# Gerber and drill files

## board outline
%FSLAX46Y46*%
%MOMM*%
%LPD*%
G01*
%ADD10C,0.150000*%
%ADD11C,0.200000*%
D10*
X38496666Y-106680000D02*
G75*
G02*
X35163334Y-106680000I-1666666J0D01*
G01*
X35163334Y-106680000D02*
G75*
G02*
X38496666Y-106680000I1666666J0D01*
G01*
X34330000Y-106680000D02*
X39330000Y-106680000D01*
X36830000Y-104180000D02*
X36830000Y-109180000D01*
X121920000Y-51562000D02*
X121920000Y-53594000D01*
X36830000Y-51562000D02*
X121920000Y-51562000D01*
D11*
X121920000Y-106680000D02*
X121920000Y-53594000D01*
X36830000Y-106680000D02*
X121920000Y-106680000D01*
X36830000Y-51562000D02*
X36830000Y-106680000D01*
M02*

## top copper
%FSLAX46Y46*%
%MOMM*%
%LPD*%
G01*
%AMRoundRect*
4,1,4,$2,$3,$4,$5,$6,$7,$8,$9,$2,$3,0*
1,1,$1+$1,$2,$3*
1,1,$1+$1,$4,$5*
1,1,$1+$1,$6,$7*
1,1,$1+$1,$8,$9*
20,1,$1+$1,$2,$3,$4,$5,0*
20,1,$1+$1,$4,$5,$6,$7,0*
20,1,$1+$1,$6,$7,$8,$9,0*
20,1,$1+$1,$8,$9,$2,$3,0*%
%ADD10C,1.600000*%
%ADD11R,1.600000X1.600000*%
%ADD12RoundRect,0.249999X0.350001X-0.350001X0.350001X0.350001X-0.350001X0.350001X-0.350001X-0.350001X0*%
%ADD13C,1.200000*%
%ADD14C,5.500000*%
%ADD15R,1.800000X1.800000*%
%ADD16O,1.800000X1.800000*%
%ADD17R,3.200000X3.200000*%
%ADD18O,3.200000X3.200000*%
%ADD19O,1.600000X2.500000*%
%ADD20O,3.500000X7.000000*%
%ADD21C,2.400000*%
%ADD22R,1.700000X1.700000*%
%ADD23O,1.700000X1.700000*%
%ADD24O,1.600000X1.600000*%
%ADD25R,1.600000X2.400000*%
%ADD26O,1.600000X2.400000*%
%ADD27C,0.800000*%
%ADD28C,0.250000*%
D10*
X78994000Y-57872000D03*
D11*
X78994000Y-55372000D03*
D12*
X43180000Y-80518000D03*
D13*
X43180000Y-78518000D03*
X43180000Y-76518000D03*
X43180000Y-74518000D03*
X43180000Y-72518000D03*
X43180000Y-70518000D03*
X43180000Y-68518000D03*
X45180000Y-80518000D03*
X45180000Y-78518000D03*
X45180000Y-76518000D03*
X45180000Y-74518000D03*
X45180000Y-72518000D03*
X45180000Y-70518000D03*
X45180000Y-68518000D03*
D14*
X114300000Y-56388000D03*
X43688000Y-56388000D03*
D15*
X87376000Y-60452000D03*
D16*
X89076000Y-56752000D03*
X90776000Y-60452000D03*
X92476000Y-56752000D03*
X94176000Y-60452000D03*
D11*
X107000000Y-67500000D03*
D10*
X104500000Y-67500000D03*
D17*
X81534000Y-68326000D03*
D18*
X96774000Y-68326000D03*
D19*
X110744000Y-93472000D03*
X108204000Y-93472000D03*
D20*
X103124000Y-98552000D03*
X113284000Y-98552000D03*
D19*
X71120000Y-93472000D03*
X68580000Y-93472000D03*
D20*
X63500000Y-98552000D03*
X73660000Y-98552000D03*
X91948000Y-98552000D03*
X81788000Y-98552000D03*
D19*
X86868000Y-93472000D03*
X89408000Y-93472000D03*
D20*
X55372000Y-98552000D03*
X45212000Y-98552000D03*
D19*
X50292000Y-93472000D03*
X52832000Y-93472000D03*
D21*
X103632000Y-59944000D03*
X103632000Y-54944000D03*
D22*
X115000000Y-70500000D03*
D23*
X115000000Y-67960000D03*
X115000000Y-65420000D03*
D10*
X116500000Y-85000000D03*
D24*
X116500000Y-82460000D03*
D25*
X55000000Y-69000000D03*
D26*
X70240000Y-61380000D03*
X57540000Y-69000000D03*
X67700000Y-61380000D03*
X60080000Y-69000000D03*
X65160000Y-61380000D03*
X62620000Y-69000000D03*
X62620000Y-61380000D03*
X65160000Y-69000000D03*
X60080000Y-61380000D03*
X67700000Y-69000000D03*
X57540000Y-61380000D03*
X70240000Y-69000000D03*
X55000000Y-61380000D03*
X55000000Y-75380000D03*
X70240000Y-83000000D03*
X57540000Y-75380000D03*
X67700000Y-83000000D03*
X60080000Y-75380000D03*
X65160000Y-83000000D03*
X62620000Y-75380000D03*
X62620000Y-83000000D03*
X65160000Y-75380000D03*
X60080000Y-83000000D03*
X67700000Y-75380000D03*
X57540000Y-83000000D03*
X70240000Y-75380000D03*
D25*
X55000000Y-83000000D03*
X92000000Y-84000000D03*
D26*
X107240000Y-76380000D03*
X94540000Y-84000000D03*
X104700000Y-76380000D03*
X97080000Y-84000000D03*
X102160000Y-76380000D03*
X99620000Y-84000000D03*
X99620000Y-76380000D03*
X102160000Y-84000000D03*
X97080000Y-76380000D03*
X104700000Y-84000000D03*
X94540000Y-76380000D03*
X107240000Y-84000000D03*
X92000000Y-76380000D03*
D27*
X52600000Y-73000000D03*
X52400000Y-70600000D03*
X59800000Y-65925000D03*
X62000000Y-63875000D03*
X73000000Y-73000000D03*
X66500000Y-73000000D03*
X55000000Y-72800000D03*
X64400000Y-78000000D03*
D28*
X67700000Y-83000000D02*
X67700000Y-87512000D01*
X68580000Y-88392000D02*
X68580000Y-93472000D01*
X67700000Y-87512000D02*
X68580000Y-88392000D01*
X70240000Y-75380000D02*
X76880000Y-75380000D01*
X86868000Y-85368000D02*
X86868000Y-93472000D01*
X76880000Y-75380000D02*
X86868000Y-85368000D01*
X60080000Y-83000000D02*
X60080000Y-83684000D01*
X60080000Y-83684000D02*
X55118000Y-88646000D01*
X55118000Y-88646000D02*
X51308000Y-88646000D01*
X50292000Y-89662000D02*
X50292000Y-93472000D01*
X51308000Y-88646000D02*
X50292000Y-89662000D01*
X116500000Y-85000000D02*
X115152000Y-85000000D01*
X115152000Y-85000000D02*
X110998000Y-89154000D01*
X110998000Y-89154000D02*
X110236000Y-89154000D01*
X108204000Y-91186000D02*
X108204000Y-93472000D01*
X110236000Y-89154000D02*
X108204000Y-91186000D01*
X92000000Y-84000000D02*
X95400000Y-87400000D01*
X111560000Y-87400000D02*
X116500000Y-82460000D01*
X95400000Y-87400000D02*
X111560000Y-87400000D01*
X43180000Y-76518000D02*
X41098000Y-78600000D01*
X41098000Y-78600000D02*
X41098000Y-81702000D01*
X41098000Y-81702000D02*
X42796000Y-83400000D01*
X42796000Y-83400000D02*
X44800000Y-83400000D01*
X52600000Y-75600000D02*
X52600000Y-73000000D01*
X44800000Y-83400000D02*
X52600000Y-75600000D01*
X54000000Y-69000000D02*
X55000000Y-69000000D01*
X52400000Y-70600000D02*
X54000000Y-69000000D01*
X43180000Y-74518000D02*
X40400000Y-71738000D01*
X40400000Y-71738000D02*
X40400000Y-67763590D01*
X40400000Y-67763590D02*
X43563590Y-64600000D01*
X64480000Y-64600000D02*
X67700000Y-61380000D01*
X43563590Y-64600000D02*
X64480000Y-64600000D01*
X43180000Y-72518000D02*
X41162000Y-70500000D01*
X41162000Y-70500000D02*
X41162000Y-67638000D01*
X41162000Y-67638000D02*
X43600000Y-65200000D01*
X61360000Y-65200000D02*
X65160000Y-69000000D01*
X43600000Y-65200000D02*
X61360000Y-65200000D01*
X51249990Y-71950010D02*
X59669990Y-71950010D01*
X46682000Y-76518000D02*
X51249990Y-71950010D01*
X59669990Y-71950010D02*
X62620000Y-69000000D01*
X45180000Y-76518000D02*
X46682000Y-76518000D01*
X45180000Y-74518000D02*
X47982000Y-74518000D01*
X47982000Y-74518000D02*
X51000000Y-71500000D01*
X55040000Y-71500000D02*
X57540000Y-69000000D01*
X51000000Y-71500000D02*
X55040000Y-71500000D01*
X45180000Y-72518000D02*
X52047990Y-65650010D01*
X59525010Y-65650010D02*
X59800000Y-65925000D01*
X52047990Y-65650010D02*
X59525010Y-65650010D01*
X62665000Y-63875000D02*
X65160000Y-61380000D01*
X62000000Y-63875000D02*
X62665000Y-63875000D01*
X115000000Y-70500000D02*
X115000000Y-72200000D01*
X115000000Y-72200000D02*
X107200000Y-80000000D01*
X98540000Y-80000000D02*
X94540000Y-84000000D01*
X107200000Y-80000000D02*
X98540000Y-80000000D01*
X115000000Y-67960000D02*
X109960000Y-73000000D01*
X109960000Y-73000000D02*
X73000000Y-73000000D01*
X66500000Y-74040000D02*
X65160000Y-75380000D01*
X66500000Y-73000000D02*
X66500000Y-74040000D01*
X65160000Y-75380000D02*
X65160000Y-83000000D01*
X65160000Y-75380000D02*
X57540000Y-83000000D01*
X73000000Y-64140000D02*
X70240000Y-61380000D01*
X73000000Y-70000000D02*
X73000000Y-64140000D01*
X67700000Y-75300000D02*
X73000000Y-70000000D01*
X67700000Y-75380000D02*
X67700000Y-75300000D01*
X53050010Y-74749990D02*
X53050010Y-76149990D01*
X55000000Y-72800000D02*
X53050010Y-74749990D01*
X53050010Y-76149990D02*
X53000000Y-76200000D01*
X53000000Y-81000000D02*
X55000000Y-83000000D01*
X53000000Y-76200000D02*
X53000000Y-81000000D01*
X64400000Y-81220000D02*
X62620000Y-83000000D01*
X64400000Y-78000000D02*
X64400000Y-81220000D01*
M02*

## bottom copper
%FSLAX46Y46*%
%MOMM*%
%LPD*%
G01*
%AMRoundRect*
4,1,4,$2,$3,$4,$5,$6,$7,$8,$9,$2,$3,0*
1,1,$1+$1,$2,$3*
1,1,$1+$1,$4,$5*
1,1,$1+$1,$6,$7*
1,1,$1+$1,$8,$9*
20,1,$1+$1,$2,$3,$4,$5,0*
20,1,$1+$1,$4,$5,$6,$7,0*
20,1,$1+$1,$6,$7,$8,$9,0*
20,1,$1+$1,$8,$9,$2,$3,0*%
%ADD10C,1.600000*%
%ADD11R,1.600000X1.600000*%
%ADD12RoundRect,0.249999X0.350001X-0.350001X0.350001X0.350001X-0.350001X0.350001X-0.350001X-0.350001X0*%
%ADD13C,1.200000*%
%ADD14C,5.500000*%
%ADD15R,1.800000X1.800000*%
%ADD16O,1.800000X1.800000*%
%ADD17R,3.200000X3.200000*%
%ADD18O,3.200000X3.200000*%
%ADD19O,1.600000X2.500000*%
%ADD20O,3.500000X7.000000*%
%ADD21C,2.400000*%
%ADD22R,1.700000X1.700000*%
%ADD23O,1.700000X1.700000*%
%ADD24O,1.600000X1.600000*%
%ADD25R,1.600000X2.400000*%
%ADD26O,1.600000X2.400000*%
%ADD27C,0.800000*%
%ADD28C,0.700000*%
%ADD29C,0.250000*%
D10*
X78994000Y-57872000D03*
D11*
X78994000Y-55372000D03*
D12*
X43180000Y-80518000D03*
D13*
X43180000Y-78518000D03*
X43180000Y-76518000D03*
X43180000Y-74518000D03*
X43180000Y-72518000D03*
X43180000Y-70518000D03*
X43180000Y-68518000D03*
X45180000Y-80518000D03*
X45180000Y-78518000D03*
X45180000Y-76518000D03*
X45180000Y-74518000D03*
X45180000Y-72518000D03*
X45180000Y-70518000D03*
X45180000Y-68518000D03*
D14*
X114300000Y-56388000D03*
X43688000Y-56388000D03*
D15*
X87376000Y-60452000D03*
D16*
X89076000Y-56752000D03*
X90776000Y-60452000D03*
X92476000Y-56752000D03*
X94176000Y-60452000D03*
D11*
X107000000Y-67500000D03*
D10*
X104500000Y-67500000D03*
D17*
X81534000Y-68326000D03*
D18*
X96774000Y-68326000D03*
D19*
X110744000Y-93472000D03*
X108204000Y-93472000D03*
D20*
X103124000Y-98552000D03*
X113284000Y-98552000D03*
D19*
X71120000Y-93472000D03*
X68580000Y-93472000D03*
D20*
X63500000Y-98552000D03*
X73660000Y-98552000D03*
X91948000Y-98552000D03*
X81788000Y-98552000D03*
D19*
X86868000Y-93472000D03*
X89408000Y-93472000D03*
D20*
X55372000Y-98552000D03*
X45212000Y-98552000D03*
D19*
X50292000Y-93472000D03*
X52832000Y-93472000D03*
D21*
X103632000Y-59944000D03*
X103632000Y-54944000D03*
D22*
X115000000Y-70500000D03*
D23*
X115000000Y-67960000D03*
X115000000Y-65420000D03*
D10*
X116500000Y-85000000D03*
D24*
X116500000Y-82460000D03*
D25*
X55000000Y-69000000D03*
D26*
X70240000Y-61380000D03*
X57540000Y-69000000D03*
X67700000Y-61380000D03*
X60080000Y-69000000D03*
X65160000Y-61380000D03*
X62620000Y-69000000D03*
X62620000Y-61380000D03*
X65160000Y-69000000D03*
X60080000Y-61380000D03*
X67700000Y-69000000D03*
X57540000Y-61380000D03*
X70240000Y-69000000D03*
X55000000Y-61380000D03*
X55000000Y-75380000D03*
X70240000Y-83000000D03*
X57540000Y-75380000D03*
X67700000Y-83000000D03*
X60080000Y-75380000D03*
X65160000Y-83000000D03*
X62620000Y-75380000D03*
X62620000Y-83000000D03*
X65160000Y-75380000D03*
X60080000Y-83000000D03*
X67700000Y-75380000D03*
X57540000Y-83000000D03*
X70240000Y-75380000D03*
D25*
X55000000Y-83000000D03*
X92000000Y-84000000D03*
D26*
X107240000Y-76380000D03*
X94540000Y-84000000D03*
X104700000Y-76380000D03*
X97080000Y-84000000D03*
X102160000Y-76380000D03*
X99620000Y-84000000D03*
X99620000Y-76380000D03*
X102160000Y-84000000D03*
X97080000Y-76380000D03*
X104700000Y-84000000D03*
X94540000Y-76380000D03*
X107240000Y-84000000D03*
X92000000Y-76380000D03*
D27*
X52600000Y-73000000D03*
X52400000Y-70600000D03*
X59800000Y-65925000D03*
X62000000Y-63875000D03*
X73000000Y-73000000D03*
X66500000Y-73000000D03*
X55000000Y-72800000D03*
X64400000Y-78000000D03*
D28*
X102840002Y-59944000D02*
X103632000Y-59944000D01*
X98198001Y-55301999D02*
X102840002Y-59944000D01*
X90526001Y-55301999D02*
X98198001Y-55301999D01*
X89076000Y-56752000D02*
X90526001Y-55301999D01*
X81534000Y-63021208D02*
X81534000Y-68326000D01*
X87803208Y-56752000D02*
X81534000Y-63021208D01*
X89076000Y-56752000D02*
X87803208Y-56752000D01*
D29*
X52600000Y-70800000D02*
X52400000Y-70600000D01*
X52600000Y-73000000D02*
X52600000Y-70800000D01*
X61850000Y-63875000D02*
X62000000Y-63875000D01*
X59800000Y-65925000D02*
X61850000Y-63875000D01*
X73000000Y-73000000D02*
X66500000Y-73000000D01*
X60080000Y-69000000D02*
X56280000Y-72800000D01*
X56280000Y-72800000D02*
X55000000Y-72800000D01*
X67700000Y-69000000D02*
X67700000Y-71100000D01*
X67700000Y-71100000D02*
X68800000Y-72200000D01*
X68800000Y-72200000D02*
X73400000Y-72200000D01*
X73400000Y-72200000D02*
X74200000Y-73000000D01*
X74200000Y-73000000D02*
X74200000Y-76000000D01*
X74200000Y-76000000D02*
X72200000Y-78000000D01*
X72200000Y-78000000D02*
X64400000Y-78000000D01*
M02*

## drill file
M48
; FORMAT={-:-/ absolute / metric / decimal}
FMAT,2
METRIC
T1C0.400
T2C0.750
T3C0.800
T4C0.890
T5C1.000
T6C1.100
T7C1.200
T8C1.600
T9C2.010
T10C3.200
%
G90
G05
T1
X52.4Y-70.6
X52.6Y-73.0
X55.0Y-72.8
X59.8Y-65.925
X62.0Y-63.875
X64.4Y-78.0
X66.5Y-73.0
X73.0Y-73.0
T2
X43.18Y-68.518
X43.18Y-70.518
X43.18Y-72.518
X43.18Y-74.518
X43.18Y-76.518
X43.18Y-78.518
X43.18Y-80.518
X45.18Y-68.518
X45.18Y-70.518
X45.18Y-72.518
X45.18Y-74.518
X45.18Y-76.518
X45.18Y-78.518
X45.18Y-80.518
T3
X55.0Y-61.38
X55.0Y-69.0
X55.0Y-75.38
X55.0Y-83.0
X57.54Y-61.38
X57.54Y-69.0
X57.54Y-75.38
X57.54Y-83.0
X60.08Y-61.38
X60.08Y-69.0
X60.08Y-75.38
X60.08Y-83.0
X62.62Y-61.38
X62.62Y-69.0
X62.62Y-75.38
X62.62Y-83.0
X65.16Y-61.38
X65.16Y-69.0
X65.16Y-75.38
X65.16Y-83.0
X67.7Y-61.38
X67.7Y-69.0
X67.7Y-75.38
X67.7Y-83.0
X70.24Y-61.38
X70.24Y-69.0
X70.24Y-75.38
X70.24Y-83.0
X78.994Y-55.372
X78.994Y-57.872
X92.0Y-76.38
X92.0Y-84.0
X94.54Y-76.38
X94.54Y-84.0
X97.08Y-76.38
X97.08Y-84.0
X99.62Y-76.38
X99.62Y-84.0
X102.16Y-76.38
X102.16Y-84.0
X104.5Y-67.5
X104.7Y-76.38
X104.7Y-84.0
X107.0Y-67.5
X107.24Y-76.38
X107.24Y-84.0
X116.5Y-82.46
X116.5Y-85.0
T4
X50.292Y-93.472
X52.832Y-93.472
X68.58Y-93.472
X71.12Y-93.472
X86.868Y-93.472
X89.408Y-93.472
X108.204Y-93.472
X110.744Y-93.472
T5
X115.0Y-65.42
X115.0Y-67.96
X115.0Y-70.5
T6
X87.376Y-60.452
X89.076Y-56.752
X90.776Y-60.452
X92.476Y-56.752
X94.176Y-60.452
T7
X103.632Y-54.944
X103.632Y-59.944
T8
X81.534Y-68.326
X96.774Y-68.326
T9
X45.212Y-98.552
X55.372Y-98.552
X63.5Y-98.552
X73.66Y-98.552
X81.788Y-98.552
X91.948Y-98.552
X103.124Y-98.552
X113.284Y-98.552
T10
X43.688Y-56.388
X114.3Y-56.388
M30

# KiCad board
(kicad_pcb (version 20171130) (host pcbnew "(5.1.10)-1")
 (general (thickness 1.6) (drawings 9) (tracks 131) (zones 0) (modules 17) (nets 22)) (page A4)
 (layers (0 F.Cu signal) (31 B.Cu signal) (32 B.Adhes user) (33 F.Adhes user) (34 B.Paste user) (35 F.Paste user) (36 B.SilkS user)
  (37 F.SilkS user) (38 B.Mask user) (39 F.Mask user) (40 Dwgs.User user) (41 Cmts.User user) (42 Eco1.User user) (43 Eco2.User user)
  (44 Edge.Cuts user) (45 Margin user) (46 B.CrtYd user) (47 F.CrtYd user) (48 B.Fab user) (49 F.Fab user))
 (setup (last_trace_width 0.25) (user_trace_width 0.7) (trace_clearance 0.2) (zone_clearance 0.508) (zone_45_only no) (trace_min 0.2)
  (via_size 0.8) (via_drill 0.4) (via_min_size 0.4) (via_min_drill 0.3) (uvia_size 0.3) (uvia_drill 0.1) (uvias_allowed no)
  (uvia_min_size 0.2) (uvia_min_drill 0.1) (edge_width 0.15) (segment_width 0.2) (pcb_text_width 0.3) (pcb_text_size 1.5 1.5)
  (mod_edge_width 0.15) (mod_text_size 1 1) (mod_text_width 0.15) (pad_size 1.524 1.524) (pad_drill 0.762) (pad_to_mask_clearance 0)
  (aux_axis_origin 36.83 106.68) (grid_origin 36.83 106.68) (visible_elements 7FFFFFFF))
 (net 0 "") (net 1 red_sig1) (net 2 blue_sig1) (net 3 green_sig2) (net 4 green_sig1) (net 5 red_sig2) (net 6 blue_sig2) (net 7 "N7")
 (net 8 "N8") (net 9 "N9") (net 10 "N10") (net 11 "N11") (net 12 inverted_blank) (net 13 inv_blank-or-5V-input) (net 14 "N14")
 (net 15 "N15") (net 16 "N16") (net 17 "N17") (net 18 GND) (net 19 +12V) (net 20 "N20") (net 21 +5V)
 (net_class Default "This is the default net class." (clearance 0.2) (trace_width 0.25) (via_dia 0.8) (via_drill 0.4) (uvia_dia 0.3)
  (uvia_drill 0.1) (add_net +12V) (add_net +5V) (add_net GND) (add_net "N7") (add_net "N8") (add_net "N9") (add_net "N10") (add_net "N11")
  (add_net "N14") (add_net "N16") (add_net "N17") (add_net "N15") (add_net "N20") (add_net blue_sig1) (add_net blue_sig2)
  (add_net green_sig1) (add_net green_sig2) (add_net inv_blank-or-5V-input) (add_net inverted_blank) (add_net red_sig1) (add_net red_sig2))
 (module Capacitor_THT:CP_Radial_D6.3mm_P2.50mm (layer F.Cu) (at 78.994 55.372 270)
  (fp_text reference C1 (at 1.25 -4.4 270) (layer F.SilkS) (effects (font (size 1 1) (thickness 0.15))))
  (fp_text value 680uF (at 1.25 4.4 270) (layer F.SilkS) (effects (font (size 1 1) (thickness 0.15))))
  (pad 2 thru_hole circle (at 2.5 0 270) (size 1.6 1.6) (drill 0.8) (layers *.Cu *.Mask))
  (pad 1 thru_hole rect (at 0 0 270) (size 1.6 1.6) (drill 0.8) (layers *.Cu *.Mask)))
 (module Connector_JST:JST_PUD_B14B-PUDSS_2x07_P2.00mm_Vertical (layer F.Cu) (at 43.18 80.518 90)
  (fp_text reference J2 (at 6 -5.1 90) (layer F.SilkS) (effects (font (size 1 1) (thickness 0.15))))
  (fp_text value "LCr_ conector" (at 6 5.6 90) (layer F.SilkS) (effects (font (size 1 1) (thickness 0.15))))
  (pad 1 thru_hole roundrect (at 0 0 90) (size 1.2 1.2) (drill 0.75) (layers *.Cu *.Mask) (roundrect_rratio 0.2083325))
  (pad 3 thru_hole circle (at 2 0 90) (size 1.2 1.2) (drill 0.75) (layers *.Cu *.Mask))
  (pad 5 thru_hole circle (at 4 0 90) (size 1.2 1.2) (drill 0.75) (layers *.Cu *.Mask) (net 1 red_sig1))
  (pad 7 thru_hole circle (at 6 0 90) (size 1.2 1.2) (drill 0.75) (layers *.Cu *.Mask) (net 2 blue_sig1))
  (pad 9 thru_hole circle (at 8 0 90) (size 1.2 1.2) (drill 0.75) (layers *.Cu *.Mask) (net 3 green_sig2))
  (pad 11 thru_hole circle (at 10 0 90) (size 1.2 1.2) (drill 0.75) (layers *.Cu *.Mask))
  (pad 13 thru_hole circle (at 12 0 90) (size 1.2 1.2) (drill 0.75) (layers *.Cu *.Mask))
  (pad 2 thru_hole circle (at 0 2 90) (size 1.2 1.2) (drill 0.75) (layers *.Cu *.Mask))
  (pad 4 thru_hole circle (at 2 2 90) (size 1.2 1.2) (drill 0.75) (layers *.Cu *.Mask))
  (pad 6 thru_hole circle (at 4 2 90) (size 1.2 1.2) (drill 0.75) (layers *.Cu *.Mask) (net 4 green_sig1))
  (pad 8 thru_hole circle (at 6 2 90) (size 1.2 1.2) (drill 0.75) (layers *.Cu *.Mask) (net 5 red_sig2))
  (pad 10 thru_hole circle (at 8 2 90) (size 1.2 1.2) (drill 0.75) (layers *.Cu *.Mask) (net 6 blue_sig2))
  (pad 12 thru_hole circle (at 10 2 90) (size 1.2 1.2) (drill 0.75) (layers *.Cu *.Mask))
  (pad 14 thru_hole circle (at 12 2 90) (size 1.2 1.2) (drill 0.75) (layers *.Cu *.Mask)))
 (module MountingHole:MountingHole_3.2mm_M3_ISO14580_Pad (layer F.Cu) (at 114.3 56.388)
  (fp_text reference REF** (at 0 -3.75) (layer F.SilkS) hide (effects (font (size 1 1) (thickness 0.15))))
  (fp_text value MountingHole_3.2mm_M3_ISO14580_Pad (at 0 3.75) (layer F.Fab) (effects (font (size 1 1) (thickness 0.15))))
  (pad 1 thru_hole circle (at 0 0) (size 5.5 5.5) (drill 3.2) (layers *.Cu *.Mask)))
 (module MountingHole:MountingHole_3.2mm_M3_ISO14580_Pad (layer F.Cu) (at 43.688 56.388)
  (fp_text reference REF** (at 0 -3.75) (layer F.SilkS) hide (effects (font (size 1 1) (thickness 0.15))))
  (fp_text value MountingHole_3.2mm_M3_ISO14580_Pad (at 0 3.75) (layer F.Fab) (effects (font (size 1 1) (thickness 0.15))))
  (pad 1 thru_hole circle (at 0 0) (size 5.5 5.5) (drill 3.2) (layers *.Cu *.Mask)))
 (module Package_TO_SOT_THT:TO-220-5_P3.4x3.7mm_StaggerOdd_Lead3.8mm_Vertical (layer F.Cu) (at 87.376 60.452)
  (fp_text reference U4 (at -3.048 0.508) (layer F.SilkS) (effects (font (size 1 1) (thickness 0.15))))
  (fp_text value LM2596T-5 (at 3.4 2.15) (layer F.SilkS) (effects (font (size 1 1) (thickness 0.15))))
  (pad 1 thru_hole rect (at 0 0) (size 1.8 1.8) (drill 1.1) (layers *.Cu *.Mask))
  (pad 2 thru_hole oval (at 1.7 -3.7) (size 1.8 1.8) (drill 1.1) (layers *.Cu *.Mask) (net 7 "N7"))
  (pad 3 thru_hole oval (at 3.4 0) (size 1.8 1.8) (drill 1.1) (layers *.Cu *.Mask))
  (pad 4 thru_hole oval (at 5.1 -3.7) (size 1.8 1.8) (drill 1.1) (layers *.Cu *.Mask))
  (pad 5 thru_hole oval (at 6.8 0) (size 1.8 1.8) (drill 1.1) (layers *.Cu *.Mask)))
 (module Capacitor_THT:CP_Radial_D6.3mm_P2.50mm (layer F.Cu) (at 107 67.5 180)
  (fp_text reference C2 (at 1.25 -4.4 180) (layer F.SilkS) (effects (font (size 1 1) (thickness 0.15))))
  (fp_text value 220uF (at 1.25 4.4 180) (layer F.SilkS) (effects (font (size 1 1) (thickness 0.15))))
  (pad 1 thru_hole rect (at 0 0 180) (size 1.6 1.6) (drill 0.8) (layers *.Cu *.Mask))
  (pad 2 thru_hole circle (at 2.5 0 180) (size 1.6 1.6) (drill 0.8) (layers *.Cu *.Mask)))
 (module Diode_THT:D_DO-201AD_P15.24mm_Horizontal (layer F.Cu) (at 81.534 68.326)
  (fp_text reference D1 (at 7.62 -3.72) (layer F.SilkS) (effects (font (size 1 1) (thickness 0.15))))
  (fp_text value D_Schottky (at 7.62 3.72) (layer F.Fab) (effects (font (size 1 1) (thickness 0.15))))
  (pad 1 thru_hole rect (at 0 0) (size 3.2 3.2) (drill 1.6) (layers *.Cu *.Mask) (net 7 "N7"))
  (pad 2 thru_hole oval (at 15.24 0) (size 3.2 3.2) (drill 1.6) (layers *.Cu *.Mask)))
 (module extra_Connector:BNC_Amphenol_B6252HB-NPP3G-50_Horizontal (layer F.Cu) (at 108.204 93.472 180)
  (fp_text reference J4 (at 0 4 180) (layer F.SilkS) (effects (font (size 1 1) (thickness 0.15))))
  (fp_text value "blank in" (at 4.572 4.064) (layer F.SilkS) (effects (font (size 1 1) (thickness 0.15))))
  (pad 2 thru_hole oval (at -2.54 0 180) (size 1.6 2.5) (drill 0.89) (layers *.Cu *.Mask))
  (pad 1 thru_hole oval (at 0 0 180) (size 1.6 2.5) (drill 0.89) (layers *.Cu *.Mask) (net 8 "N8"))
  (pad 2 thru_hole oval (at 5.08 -5.08 180) (size 3.5 7) (drill 2.01) (layers *.Cu *.Mask))
  (pad 2 thru_hole oval (at -5.08 -5.08 180) (size 3.5 7) (drill 2.01) (layers *.Cu *.Mask)))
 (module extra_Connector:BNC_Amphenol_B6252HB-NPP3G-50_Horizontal (layer F.Cu) (at 68.58 93.472 180)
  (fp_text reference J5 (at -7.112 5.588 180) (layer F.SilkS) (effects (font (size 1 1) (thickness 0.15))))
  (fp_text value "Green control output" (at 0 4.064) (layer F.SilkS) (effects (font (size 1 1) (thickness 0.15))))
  (pad 2 thru_hole oval (at -2.54 0 180) (size 1.6 2.5) (drill 0.89) (layers *.Cu *.Mask))
  (pad 1 thru_hole oval (at 0 0 180) (size 1.6 2.5) (drill 0.89) (layers *.Cu *.Mask) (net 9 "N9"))
  (pad 2 thru_hole oval (at 5.08 -5.08 180) (size 3.5 7) (drill 2.01) (layers *.Cu *.Mask))
  (pad 2 thru_hole oval (at -5.08 -5.08 180) (size 3.5 7) (drill 2.01) (layers *.Cu *.Mask)))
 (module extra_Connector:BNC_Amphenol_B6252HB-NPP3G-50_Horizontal (layer F.Cu) (at 86.868 93.472 180)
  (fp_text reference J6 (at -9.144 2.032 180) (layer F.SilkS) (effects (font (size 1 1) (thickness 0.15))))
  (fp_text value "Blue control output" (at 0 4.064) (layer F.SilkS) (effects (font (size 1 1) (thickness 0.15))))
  (pad 2 thru_hole oval (at -5.08 -5.08 180) (size 3.5 7) (drill 2.01) (layers *.Cu *.Mask))
  (pad 2 thru_hole oval (at 5.08 -5.08 180) (size 3.5 7) (drill 2.01) (layers *.Cu *.Mask))
  (pad 1 thru_hole oval (at 0 0 180) (size 1.6 2.5) (drill 0.89) (layers *.Cu *.Mask) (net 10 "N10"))
  (pad 2 thru_hole oval (at -2.54 0 180) (size 1.6 2.5) (drill 0.89) (layers *.Cu *.Mask)))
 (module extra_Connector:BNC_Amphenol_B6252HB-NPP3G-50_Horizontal (layer F.Cu) (at 50.292 93.472 180)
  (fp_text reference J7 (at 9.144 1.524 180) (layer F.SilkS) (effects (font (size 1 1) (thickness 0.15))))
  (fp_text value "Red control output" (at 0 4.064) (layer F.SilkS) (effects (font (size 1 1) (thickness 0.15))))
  (pad 2 thru_hole oval (at -5.08 -5.08 180) (size 3.5 7) (drill 2.01) (layers *.Cu *.Mask))
  (pad 2 thru_hole oval (at 5.08 -5.08 180) (size 3.5 7) (drill 2.01) (layers *.Cu *.Mask))
  (pad 1 thru_hole oval (at 0 0 180) (size 1.6 2.5) (drill 0.89) (layers *.Cu *.Mask) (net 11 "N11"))
  (pad 2 thru_hole oval (at -2.54 0 180) (size 1.6 2.5) (drill 0.89) (layers *.Cu *.Mask)))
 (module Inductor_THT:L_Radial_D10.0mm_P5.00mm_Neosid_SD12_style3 (layer F.Cu) (at 103.632 59.944 90)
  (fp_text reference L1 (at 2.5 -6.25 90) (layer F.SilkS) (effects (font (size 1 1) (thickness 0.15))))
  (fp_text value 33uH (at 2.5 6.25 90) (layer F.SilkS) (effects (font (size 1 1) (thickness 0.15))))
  (pad 1 thru_hole circle (at 0 0 90) (size 2.4 2.4) (drill 1.2) (layers *.Cu *.Mask) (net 7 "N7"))
  (pad 2 thru_hole circle (at 5 0 90) (size 2.4 2.4) (drill 1.2) (layers *.Cu *.Mask)))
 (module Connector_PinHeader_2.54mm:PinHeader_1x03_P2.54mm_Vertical (layer F.Cu) (at 115 70.5 180)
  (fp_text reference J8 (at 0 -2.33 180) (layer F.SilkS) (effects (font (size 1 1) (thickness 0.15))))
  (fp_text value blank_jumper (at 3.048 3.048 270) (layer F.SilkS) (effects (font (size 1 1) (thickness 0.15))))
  (pad 1 thru_hole rect (at 0 0 180) (size 1.7 1.7) (drill 1) (layers *.Cu *.Mask) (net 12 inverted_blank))
  (pad 2 thru_hole oval (at 0 2.54 180) (size 1.7 1.7) (drill 1) (layers *.Cu *.Mask) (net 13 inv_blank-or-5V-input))
  (pad 3 thru_hole oval (at 0 5.08 180) (size 1.7 1.7) (drill 1) (layers *.Cu *.Mask)))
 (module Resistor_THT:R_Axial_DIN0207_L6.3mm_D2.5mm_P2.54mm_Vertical (layer F.Cu) (at 116.5 85 90)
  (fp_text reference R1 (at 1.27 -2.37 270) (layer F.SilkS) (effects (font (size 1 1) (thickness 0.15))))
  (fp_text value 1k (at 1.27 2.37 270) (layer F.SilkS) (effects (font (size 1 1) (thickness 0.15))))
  (pad 1 thru_hole circle (at 0 0 90) (size 1.6 1.6) (drill 0.8) (layers *.Cu *.Mask) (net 8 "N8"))
  (pad 2 thru_hole oval (at 2.54 0 90) (size 1.6 1.6) (drill 0.8) (layers *.Cu *.Mask) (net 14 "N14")))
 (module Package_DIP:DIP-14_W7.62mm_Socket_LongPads (layer F.Cu) (at 55 69 90)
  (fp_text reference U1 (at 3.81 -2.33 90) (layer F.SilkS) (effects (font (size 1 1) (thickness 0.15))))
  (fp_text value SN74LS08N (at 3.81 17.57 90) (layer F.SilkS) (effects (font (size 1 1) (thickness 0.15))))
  (pad 1 thru_hole rect (at 0 0 90) (size 2.4 1.6) (drill 0.8) (layers *.Cu *.Mask) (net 1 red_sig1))
  (pad 8 thru_hole oval (at 7.62 15.24 90) (size 2.4 1.6) (drill 0.8) (layers *.Cu *.Mask) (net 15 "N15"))
  (pad 2 thru_hole oval (at 0 2.54 90) (size 2.4 1.6) (drill 0.8) (layers *.Cu *.Mask) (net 5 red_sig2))
  (pad 9 thru_hole oval (at 7.62 12.7 90) (size 2.4 1.6) (drill 0.8) (layers *.Cu *.Mask) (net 2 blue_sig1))
  (pad 3 thru_hole oval (at 0 5.08 90) (size 2.4 1.6) (drill 0.8) (layers *.Cu *.Mask) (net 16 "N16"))
  (pad 10 thru_hole oval (at 7.62 10.16 90) (size 2.4 1.6) (drill 0.8) (layers *.Cu *.Mask) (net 6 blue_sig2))
  (pad 4 thru_hole oval (at 0 7.62 90) (size 2.4 1.6) (drill 0.8) (layers *.Cu *.Mask) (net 4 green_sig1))
  (pad 11 thru_hole oval (at 7.62 7.62 90) (size 2.4 1.6) (drill 0.8) (layers *.Cu *.Mask))
  (pad 5 thru_hole oval (at 0 10.16 90) (size 2.4 1.6) (drill 0.8) (layers *.Cu *.Mask) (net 3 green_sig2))
  (pad 12 thru_hole oval (at 7.62 5.08 90) (size 2.4 1.6) (drill 0.8) (layers *.Cu *.Mask))
  (pad 6 thru_hole oval (at 0 12.7 90) (size 2.4 1.6) (drill 0.8) (layers *.Cu *.Mask) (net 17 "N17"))
  (pad 13 thru_hole oval (at 7.62 2.54 90) (size 2.4 1.6) (drill 0.8) (layers *.Cu *.Mask))
  (pad 7 thru_hole oval (at 0 15.24 90) (size 2.4 1.6) (drill 0.8) (layers *.Cu *.Mask))
  (pad 14 thru_hole oval (at 7.62 0 90) (size 2.4 1.6) (drill 0.8) (layers *.Cu *.Mask)))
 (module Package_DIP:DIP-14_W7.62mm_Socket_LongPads (layer F.Cu) (at 55 83 90)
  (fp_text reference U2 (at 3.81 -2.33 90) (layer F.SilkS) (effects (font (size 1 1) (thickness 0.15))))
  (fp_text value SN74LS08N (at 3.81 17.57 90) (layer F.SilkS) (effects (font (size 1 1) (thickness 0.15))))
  (pad 14 thru_hole oval (at 7.62 0 90) (size 2.4 1.6) (drill 0.8) (layers *.Cu *.Mask))
  (pad 7 thru_hole oval (at 0 15.24 90) (size 2.4 1.6) (drill 0.8) (layers *.Cu *.Mask))
  (pad 13 thru_hole oval (at 7.62 2.54 90) (size 2.4 1.6) (drill 0.8) (layers *.Cu *.Mask))
  (pad 6 thru_hole oval (at 0 12.7 90) (size 2.4 1.6) (drill 0.8) (layers *.Cu *.Mask) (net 9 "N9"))
  (pad 12 thru_hole oval (at 7.62 5.08 90) (size 2.4 1.6) (drill 0.8) (layers *.Cu *.Mask))
  (pad 5 thru_hole oval (at 0 10.16 90) (size 2.4 1.6) (drill 0.8) (layers *.Cu *.Mask) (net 13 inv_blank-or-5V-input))
  (pad 11 thru_hole oval (at 7.62 7.62 90) (size 2.4 1.6) (drill 0.8) (layers *.Cu *.Mask))
  (pad 4 thru_hole oval (at 0 7.62 90) (size 2.4 1.6) (drill 0.8) (layers *.Cu *.Mask) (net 17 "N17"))
  (pad 10 thru_hole oval (at 7.62 10.16 90) (size 2.4 1.6) (drill 0.8) (layers *.Cu *.Mask) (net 13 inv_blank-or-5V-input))
  (pad 3 thru_hole oval (at 0 5.08 90) (size 2.4 1.6) (drill 0.8) (layers *.Cu *.Mask) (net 11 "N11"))
  (pad 9 thru_hole oval (at 7.62 12.7 90) (size 2.4 1.6) (drill 0.8) (layers *.Cu *.Mask) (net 15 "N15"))
  (pad 2 thru_hole oval (at 0 2.54 90) (size 2.4 1.6) (drill 0.8) (layers *.Cu *.Mask) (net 13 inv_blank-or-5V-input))
  (pad 8 thru_hole oval (at 7.62 15.24 90) (size 2.4 1.6) (drill 0.8) (layers *.Cu *.Mask) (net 10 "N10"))
  (pad 1 thru_hole rect (at 0 0 90) (size 2.4 1.6) (drill 0.8) (layers *.Cu *.Mask) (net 16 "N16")))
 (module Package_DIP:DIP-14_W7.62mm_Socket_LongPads (layer F.Cu) (at 92 84 90)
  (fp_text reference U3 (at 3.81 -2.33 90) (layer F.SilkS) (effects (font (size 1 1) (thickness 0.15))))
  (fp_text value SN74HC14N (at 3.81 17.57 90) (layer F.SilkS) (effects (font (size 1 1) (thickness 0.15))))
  (pad 1 thru_hole rect (at 0 0 90) (size 2.4 1.6) (drill 0.8) (layers *.Cu *.Mask) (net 14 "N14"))
  (pad 8 thru_hole oval (at 7.62 15.24 90) (size 2.4 1.6) (drill 0.8) (layers *.Cu *.Mask))
  (pad 2 thru_hole oval (at 0 2.54 90) (size 2.4 1.6) (drill 0.8) (layers *.Cu *.Mask) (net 12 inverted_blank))
  (pad 9 thru_hole oval (at 7.62 12.7 90) (size 2.4 1.6) (drill 0.8) (layers *.Cu *.Mask))
  (pad 3 thru_hole oval (at 0 5.08 90) (size 2.4 1.6) (drill 0.8) (layers *.Cu *.Mask))
  (pad 10 thru_hole oval (at 7.62 10.16 90) (size 2.4 1.6) (drill 0.8) (layers *.Cu *.Mask))
  (pad 4 thru_hole oval (at 0 7.62 90) (size 2.4 1.6) (drill 0.8) (layers *.Cu *.Mask))
  (pad 11 thru_hole oval (at 7.62 7.62 90) (size 2.4 1.6) (drill 0.8) (layers *.Cu *.Mask))
  (pad 5 thru_hole oval (at 0 10.16 90) (size 2.4 1.6) (drill 0.8) (layers *.Cu *.Mask))
  (pad 12 thru_hole oval (at 7.62 5.08 90) (size 2.4 1.6) (drill 0.8) (layers *.Cu *.Mask))
  (pad 6 thru_hole oval (at 0 12.7 90) (size 2.4 1.6) (drill 0.8) (layers *.Cu *.Mask))
  (pad 13 thru_hole oval (at 7.62 2.54 90) (size 2.4 1.6) (drill 0.8) (layers *.Cu *.Mask))
  (pad 7 thru_hole oval (at 0 15.24 90) (size 2.4 1.6) (drill 0.8) (layers *.Cu *.Mask))
  (pad 14 thru_hole oval (at 7.62 0 90) (size 2.4 1.6) (drill 0.8) (layers *.Cu *.Mask)))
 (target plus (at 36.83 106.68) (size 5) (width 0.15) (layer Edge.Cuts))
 (gr_line (start 121.92 51.562) (end 121.92 53.594) (layer Edge.Cuts) (width 0.15))
 (gr_line (start 36.83 51.562) (end 121.92 51.562) (layer Edge.Cuts) (width 0.15))
 (gr_line (start 121.92 106.68) (end 121.92 53.594) (layer Edge.Cuts) (width 0.2))
 (gr_line (start 36.83 106.68) (end 121.92 106.68) (layer Edge.Cuts) (width 0.2))
 (gr_line (start 36.83 51.562) (end 36.83 106.68) (layer Edge.Cuts) (width 0.2))
 (segment (start 102.840002 59.944) (end 103.632 59.944) (width 0.7) (layer B.Cu) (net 7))
 (segment (start 98.198001 55.301999) (end 102.840002 59.944) (width 0.7) (layer B.Cu) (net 7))
 (segment (start 90.526001 55.301999) (end 98.198001 55.301999) (width 0.7) (layer B.Cu) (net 7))
 (segment (start 89.076 56.752) (end 90.526001 55.301999) (width 0.7) (layer B.Cu) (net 7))
 (segment (start 81.534 63.021208) (end 81.534 68.326) (width 0.7) (layer B.Cu) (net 7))
 (segment (start 87.803208 56.752) (end 81.534 63.021208) (width 0.7) (layer B.Cu) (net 7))
 (segment (start 89.076 56.752) (end 87.803208 56.752) (width 0.7) (layer B.Cu) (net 7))
 (segment (start 67.7 83) (end 67.7 87.512) (width 0.25) (layer F.Cu) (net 9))
 (segment (start 68.58 88.392) (end 68.58 93.472) (width 0.25) (layer F.Cu) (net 9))
 (segment (start 67.7 87.512) (end 68.58 88.392) (width 0.25) (layer F.Cu) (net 9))
 (segment (start 70.24 75.38) (end 76.88 75.38) (width 0.25) (layer F.Cu) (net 10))
 (segment (start 86.868 85.368) (end 86.868 93.472) (width 0.25) (layer F.Cu) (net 10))
 (segment (start 76.88 75.38) (end 86.868 85.368) (width 0.25) (layer F.Cu) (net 10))
 (segment (start 60.08 83) (end 60.08 83.684) (width 0.25) (layer F.Cu) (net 11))
 (segment (start 60.08 83.684) (end 55.118 88.646) (width 0.25) (layer F.Cu) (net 11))
 (segment (start 55.118 88.646) (end 51.308 88.646) (width 0.25) (layer F.Cu) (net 11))
 (segment (start 50.292 89.662) (end 50.292 93.472) (width 0.25) (layer F.Cu) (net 11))
 (segment (start 51.308 88.646) (end 50.292 89.662) (width 0.25) (layer F.Cu) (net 11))
 (segment (start 116.5 85) (end 115.152 85) (width 0.25) (layer F.Cu) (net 8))
 (segment (start 115.152 85) (end 110.998 89.154) (width 0.25) (layer F.Cu) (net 8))
 (segment (start 110.998 89.154) (end 110.236 89.154) (width 0.25) (layer F.Cu) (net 8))
 (segment (start 108.204 91.186) (end 108.204 93.472) (width 0.25) (layer F.Cu) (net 8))
 (segment (start 110.236 89.154) (end 108.204 91.186) (width 0.25) (layer F.Cu) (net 8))
 (segment (start 92 84) (end 95.4 87.4) (width 0.25) (layer F.Cu) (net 14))
 (segment (start 111.56 87.4) (end 116.5 82.46) (width 0.25) (layer F.Cu) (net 14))
 (segment (start 95.4 87.4) (end 111.56 87.4) (width 0.25) (layer F.Cu) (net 14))
 (segment (start 43.18 76.518) (end 41.098 78.6) (width 0.25) (layer F.Cu) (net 1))
 (segment (start 41.098 78.6) (end 41.098 81.702) (width 0.25) (layer F.Cu) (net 1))
 (segment (start 41.098 81.702) (end 42.796 83.4) (width 0.25) (layer F.Cu) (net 1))
 (segment (start 42.796 83.4) (end 44.8 83.4) (width 0.25) (layer F.Cu) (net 1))
 (segment (start 52.6 75.6) (end 52.6 73) (width 0.25) (layer F.Cu) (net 1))
 (segment (start 44.8 83.4) (end 52.6 75.6) (width 0.25) (layer F.Cu) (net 1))
 (segment (start 52.6 70.8) (end 52.4 70.6) (width 0.25) (layer B.Cu) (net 1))
 (segment (start 52.6 73) (end 52.6 70.8) (width 0.25) (layer B.Cu) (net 1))
 (segment (start 54 69) (end 55 69) (width 0.25) (layer F.Cu) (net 1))
 (segment (start 52.4 70.6) (end 54 69) (width 0.25) (layer F.Cu) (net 1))
 (segment (start 43.18 74.518) (end 40.4 71.738) (width 0.25) (layer F.Cu) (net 2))
 (segment (start 40.4 71.738) (end 40.4 67.76359) (width 0.25) (layer F.Cu) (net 2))
 (segment (start 40.4 67.76359) (end 43.56359 64.6) (width 0.25) (layer F.Cu) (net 2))
 (segment (start 64.48 64.6) (end 67.7 61.38) (width 0.25) (layer F.Cu) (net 2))
 (segment (start 43.56359 64.6) (end 64.48 64.6) (width 0.25) (layer F.Cu) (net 2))
 (segment (start 43.18 72.518) (end 41.162 70.5) (width 0.25) (layer F.Cu) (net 3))
 (segment (start 41.162 70.5) (end 41.162 67.638) (width 0.25) (layer F.Cu) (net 3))
 (segment (start 41.162 67.638) (end 43.6 65.2) (width 0.25) (layer F.Cu) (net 3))
 (segment (start 61.36 65.2) (end 65.16 69) (width 0.25) (layer F.Cu) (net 3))
 (segment (start 43.6 65.2) (end 61.36 65.2) (width 0.25) (layer F.Cu) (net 3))
 (segment (start 51.24999 71.95001) (end 59.66999 71.95001) (width 0.25) (layer F.Cu) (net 4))
 (segment (start 46.682 76.518) (end 51.24999 71.95001) (width 0.25) (layer F.Cu) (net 4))
 (segment (start 59.66999 71.95001) (end 62.62 69) (width 0.25) (layer F.Cu) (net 4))
 (segment (start 45.18 76.518) (end 46.682 76.518) (width 0.25) (layer F.Cu) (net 4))
 (segment (start 45.18 74.518) (end 47.982 74.518) (width 0.25) (layer F.Cu) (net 5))
 (segment (start 47.982 74.518) (end 51 71.5) (width 0.25) (layer F.Cu) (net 5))
 (segment (start 55.04 71.5) (end 57.54 69) (width 0.25) (layer F.Cu) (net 5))
 (segment (start 51 71.5) (end 55.04 71.5) (width 0.25) (layer F.Cu) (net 5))
 (segment (start 45.18 72.518) (end 52.04799 65.65001) (width 0.25) (layer F.Cu) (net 6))
 (segment (start 59.52501 65.65001) (end 59.8 65.925) (width 0.25) (layer F.Cu) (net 6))
 (segment (start 52.04799 65.65001) (end 59.52501 65.65001) (width 0.25) (layer F.Cu) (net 6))
 (segment (start 61.85 63.875) (end 62 63.875) (width 0.25) (layer B.Cu) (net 6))
 (segment (start 59.8 65.925) (end 61.85 63.875) (width 0.25) (layer B.Cu) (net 6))
 (segment (start 62.665 63.875) (end 65.16 61.38) (width 0.25) (layer F.Cu) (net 6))
 (segment (start 62 63.875) (end 62.665 63.875) (width 0.25) (layer F.Cu) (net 6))
 (segment (start 115 70.5) (end 115 72.2) (width 0.25) (layer F.Cu) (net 12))
 (segment (start 115 72.2) (end 107.2 80) (width 0.25) (layer F.Cu) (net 12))
 (segment (start 98.54 80) (end 94.54 84) (width 0.25) (layer F.Cu) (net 12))
 (segment (start 107.2 80) (end 98.54 80) (width 0.25) (layer F.Cu) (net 12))
 (segment (start 115 67.96) (end 109.96 73) (width 0.25) (layer F.Cu) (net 13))
 (segment (start 109.96 73) (end 73 73) (width 0.25) (layer F.Cu) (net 13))
 (segment (start 73 73) (end 66.5 73) (width 0.25) (layer B.Cu) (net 13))
 (segment (start 66.5 74.04) (end 65.16 75.38) (width 0.25) (layer F.Cu) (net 13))
 (segment (start 66.5 73) (end 66.5 74.04) (width 0.25) (layer F.Cu) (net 13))
 (segment (start 65.16 75.38) (end 65.16 83) (width 0.25) (layer F.Cu) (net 13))
 (segment (start 65.16 75.38) (end 57.54 83) (width 0.25) (layer F.Cu) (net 13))
 (segment (start 73 64.14) (end 70.24 61.38) (width 0.25) (layer F.Cu) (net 15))
 (segment (start 73 70) (end 73 64.14) (width 0.25) (layer F.Cu) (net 15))
 (segment (start 67.7 75.3) (end 73 70) (width 0.25) (layer F.Cu) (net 15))
 (segment (start 67.7 75.38) (end 67.7 75.3) (width 0.25) (layer F.Cu) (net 15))
 (segment (start 60.08 69) (end 56.28 72.8) (width 0.25) (layer B.Cu) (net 16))
 (segment (start 56.28 72.8) (end 55 72.8) (width 0.25) (layer B.Cu) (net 16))
 (segment (start 53.05001 74.74999) (end 53.05001 76.14999) (width 0.25) (layer F.Cu) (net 16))
 (segment (start 55 72.8) (end 53.05001 74.74999) (width 0.25) (layer F.Cu) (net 16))
 (segment (start 53.05001 76.14999) (end 53 76.2) (width 0.25) (layer F.Cu) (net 16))
 (segment (start 53 81) (end 55 83) (width 0.25) (layer F.Cu) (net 16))
 (segment (start 53 76.2) (end 53 81) (width 0.25) (layer F.Cu) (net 16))
 (segment (start 67.7 69) (end 67.7 71.1) (width 0.25) (layer B.Cu) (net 17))
 (segment (start 67.7 71.1) (end 68.8 72.2) (width 0.25) (layer B.Cu) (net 17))
 (segment (start 68.8 72.2) (end 73.4 72.2) (width 0.25) (layer B.Cu) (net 17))
 (segment (start 73.4 72.2) (end 74.2 73) (width 0.25) (layer B.Cu) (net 17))
 (segment (start 74.2 73) (end 74.2 76) (width 0.25) (layer B.Cu) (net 17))
 (segment (start 74.2 76) (end 72.2 78) (width 0.25) (layer B.Cu) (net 17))
 (segment (start 72.2 78) (end 64.4 78) (width 0.25) (layer B.Cu) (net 17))
 (segment (start 64.4 81.22) (end 62.62 83) (width 0.25) (layer F.Cu) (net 17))
 (segment (start 64.4 78) (end 64.4 81.22) (width 0.25) (layer F.Cu) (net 17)) (via (at 52.6 73) (size 0.8) (layers F.Cu B.Cu) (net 1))
 (via (at 52.4 70.6) (size 0.8) (layers F.Cu B.Cu) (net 1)) (via (at 59.8 65.925) (size 0.8) (layers F.Cu B.Cu) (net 6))
 (via (at 62 63.875) (size 0.8) (layers F.Cu B.Cu) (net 6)) (via (at 73 73) (size 0.8) (layers F.Cu B.Cu) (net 13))
 (via (at 66.5 73) (size 0.8) (layers F.Cu B.Cu) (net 13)) (via (at 55 72.8) (size 0.8) (layers F.Cu B.Cu) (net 16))
 (via (at 64.4 78) (size 0.8) (layers F.Cu B.Cu) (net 17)))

